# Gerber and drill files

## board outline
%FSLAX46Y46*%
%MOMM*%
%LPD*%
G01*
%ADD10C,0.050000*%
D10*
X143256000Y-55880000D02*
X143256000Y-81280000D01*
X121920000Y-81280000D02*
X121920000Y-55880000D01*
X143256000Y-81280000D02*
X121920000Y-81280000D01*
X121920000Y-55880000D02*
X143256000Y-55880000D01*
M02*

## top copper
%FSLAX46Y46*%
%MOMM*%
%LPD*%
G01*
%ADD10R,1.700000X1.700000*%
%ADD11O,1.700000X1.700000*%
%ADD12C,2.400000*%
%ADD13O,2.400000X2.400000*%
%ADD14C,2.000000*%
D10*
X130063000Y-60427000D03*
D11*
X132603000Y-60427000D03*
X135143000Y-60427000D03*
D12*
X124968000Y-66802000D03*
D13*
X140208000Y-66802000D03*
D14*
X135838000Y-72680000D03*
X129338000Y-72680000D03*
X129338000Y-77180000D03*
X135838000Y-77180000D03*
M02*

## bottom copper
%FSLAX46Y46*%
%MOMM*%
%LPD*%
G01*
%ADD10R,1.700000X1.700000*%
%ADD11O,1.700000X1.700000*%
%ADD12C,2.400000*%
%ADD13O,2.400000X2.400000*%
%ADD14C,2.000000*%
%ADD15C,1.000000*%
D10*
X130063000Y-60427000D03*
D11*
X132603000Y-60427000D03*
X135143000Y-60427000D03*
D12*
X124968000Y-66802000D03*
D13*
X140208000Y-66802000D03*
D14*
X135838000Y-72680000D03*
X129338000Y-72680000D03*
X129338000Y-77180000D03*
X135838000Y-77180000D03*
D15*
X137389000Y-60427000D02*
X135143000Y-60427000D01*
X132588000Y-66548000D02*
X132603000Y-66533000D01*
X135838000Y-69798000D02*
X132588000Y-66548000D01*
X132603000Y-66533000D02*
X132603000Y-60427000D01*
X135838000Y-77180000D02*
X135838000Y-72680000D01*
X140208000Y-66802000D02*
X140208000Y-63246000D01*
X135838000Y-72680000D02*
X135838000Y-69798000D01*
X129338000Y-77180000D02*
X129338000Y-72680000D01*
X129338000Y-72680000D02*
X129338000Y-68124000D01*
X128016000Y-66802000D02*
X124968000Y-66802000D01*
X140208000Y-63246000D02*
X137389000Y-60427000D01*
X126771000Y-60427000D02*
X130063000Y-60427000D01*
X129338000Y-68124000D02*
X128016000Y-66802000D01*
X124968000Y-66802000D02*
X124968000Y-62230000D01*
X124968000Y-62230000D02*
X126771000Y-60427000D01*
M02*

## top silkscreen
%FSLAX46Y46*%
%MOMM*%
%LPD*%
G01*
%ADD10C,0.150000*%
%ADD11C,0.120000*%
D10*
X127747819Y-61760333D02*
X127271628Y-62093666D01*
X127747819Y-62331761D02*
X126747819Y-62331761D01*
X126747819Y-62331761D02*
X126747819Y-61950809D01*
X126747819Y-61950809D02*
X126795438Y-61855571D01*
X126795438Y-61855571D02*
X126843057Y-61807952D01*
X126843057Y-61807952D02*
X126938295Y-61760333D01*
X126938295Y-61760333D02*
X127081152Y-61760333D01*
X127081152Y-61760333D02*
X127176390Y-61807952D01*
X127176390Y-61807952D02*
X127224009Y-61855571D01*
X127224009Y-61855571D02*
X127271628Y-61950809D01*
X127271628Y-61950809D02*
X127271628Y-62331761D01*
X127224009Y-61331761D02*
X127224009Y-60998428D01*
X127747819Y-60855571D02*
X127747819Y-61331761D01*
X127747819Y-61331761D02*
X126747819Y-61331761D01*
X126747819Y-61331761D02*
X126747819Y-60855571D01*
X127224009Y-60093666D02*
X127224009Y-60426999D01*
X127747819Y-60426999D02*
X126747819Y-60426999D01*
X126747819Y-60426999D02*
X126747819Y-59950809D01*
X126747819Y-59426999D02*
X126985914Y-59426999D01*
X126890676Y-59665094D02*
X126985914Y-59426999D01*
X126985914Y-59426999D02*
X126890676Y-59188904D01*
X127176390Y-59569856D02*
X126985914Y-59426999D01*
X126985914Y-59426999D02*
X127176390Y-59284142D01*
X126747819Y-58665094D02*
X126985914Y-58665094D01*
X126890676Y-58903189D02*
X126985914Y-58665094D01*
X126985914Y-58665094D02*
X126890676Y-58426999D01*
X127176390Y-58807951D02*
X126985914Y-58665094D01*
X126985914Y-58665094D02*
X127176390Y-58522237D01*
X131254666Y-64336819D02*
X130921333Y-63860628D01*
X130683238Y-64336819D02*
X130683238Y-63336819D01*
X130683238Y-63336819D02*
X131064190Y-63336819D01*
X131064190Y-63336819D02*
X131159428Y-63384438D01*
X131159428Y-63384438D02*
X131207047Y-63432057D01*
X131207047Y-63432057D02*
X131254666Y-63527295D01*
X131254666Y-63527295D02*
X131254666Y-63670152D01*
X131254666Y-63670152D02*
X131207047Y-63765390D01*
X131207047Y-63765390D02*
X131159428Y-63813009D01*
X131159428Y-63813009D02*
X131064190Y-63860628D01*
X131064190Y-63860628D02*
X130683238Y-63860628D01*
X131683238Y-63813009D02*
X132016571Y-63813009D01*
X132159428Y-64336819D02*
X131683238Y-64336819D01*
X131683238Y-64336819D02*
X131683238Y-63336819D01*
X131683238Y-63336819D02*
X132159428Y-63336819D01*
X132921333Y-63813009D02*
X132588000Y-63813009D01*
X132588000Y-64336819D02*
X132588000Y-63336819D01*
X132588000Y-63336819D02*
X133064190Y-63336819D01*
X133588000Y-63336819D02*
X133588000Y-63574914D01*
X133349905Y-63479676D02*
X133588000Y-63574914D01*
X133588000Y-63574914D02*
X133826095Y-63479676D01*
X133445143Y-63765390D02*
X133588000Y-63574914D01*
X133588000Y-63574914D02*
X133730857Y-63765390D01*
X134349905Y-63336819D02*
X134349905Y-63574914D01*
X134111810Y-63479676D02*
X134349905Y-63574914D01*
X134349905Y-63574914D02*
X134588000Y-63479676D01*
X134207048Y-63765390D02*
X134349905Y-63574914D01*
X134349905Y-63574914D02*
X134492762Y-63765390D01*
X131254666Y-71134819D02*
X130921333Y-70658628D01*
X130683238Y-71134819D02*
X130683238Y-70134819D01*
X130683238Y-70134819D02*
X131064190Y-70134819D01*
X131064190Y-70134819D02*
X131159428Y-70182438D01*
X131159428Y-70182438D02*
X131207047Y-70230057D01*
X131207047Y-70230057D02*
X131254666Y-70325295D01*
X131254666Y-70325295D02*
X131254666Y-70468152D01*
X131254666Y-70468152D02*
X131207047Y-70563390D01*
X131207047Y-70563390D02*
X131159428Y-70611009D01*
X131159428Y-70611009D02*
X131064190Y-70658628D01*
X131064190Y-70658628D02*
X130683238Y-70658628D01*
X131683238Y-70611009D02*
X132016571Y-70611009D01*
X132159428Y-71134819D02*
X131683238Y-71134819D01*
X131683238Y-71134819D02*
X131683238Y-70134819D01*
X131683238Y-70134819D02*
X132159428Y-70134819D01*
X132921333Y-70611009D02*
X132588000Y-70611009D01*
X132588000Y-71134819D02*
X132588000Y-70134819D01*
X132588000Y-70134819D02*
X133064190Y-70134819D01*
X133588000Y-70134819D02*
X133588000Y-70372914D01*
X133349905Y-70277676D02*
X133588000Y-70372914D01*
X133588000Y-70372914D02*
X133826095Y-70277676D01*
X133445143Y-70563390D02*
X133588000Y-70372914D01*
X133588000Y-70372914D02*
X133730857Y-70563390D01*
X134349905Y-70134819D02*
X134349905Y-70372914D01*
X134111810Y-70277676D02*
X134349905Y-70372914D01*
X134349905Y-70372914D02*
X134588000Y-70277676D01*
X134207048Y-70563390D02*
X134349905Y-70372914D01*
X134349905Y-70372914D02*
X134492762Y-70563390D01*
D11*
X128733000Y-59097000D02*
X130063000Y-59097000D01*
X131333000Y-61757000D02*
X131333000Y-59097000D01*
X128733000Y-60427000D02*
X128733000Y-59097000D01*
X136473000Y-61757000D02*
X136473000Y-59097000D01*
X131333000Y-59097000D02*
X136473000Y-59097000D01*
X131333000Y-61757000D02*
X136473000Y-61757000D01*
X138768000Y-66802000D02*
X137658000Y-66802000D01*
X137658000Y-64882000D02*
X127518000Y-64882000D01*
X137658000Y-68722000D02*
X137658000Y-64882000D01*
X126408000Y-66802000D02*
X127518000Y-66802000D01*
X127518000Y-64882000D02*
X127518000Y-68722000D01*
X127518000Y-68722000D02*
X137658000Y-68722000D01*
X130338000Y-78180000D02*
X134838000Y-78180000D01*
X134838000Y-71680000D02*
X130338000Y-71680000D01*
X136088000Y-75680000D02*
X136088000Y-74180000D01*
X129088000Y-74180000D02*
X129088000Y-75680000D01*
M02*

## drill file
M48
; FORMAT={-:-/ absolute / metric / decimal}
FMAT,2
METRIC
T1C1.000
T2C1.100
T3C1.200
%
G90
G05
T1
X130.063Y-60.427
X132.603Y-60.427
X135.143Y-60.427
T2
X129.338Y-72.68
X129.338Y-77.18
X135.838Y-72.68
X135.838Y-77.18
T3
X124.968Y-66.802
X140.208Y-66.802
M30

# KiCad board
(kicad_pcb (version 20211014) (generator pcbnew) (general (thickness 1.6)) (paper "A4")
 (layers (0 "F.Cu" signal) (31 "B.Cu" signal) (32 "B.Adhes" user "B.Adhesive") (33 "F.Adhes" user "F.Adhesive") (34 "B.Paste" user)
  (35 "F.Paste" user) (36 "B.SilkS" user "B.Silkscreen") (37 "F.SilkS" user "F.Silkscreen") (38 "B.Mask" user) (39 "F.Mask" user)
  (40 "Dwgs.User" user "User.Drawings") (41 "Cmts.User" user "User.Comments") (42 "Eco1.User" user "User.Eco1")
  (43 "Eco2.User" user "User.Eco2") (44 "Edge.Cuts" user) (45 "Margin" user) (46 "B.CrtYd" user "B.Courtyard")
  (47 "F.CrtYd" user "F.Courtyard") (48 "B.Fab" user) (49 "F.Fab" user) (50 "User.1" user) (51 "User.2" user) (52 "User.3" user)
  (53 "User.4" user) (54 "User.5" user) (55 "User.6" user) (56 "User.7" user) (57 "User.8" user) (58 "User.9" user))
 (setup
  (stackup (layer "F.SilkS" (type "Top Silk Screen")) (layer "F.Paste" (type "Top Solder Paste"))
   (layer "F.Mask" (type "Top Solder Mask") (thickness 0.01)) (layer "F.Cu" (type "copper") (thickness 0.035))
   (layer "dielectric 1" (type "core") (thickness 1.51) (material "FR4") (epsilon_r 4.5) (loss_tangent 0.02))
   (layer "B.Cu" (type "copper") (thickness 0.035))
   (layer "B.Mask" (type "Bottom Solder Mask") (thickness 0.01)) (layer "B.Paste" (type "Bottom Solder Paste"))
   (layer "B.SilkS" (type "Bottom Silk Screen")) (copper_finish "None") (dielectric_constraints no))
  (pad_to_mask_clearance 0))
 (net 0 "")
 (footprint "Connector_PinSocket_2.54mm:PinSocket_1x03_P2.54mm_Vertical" (layer "F.Cu") (at 130.063 60.427 90)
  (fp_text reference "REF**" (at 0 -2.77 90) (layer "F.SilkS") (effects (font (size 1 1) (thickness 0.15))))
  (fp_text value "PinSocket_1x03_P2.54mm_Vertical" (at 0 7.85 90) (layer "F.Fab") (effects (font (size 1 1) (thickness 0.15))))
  (fp_line (start 1.33 -1.33) (end 1.33 0) (layer "F.SilkS") (width 0.12))
  (fp_line (start -1.33 1.27) (end 1.33 1.27) (layer "F.SilkS") (width 0.12))
  (fp_line (start 0 -1.33) (end 1.33 -1.33) (layer "F.SilkS") (width 0.12))
  (fp_line (start -1.33 6.41) (end 1.33 6.41) (layer "F.SilkS") (width 0.12))
  (fp_line (start 1.33 1.27) (end 1.33 6.41) (layer "F.SilkS") (width 0.12))
  (fp_line (start -1.33 1.27) (end -1.33 6.41) (layer "F.SilkS") (width 0.12))
  (pad "1" thru_hole rect (at 0 0 90) (size 1.7 1.7) (drill 1) (layers *.Cu *.Mask))
  (pad "2" thru_hole oval (at 0 2.54 90) (size 1.7 1.7) (drill 1) (layers *.Cu *.Mask))
  (pad "3" thru_hole oval (at 0 5.08 90) (size 1.7 1.7) (drill 1) (layers *.Cu *.Mask)))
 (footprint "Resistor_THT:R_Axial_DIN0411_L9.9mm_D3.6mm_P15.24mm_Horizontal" (layer "F.Cu") (at 124.968 66.802)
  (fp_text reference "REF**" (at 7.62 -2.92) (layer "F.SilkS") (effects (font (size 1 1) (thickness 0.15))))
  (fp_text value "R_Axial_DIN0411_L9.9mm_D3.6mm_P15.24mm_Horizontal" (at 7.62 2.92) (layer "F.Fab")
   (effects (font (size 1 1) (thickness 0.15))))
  (fp_line (start 13.8 0) (end 12.69 0) (layer "F.SilkS") (width 0.12))
  (fp_line (start 12.69 -1.92) (end 2.55 -1.92) (layer "F.SilkS") (width 0.12))
  (fp_line (start 12.69 1.92) (end 12.69 -1.92) (layer "F.SilkS") (width 0.12))
  (fp_line (start 1.44 0) (end 2.55 0) (layer "F.SilkS") (width 0.12))
  (fp_line (start 2.55 -1.92) (end 2.55 1.92) (layer "F.SilkS") (width 0.12))
  (fp_line (start 2.55 1.92) (end 12.69 1.92) (layer "F.SilkS") (width 0.12))
  (pad "1" thru_hole circle (at 0 0) (size 2.4 2.4) (drill 1.2) (layers *.Cu *.Mask))
  (pad "2" thru_hole oval (at 15.24 0) (size 2.4 2.4) (drill 1.2) (layers *.Cu *.Mask)))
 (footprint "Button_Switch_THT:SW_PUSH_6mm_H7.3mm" (layer "F.Cu") (at 129.338 72.68)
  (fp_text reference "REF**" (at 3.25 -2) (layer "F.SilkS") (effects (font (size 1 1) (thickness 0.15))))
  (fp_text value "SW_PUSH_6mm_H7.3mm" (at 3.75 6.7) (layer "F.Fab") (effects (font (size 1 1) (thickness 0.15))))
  (fp_line (start 1 5.5) (end 5.5 5.5) (layer "F.SilkS") (width 0.12))
  (fp_line (start 5.5 -1) (end 1 -1) (layer "F.SilkS") (width 0.12))
  (fp_line (start 6.75 3) (end 6.75 1.5) (layer "F.SilkS") (width 0.12))
  (fp_line (start -0.25 1.5) (end -0.25 3) (layer "F.SilkS") (width 0.12))
  (pad "1" thru_hole circle (at 6.5 0 90) (size 2 2) (drill 1.1) (layers *.Cu *.Mask))
  (pad "1" thru_hole circle (at 0 0 90) (size 2 2) (drill 1.1) (layers *.Cu *.Mask))
  (pad "2" thru_hole circle (at 0 4.5 90) (size 2 2) (drill 1.1) (layers *.Cu *.Mask))
  (pad "2" thru_hole circle (at 6.5 4.5 90) (size 2 2) (drill 1.1) (layers *.Cu *.Mask)))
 (gr_line (start 143.256 55.88) (end 143.256 81.28) (layer "Edge.Cuts") (width 0.05))
 (gr_line (start 121.92 81.28) (end 121.92 55.88) (layer "Edge.Cuts") (width 0.05))
 (gr_line (start 143.256 81.28) (end 121.92 81.28) (layer "Edge.Cuts") (width 0.05))
 (gr_line (start 121.92 55.88) (end 143.256 55.88) (layer "Edge.Cuts") (width 0.05))
 (segment (start 137.389 60.427) (end 135.143 60.427) (width 1) (layer "B.Cu") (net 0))
 (segment (start 132.588 66.548) (end 132.603 66.533) (width 1) (layer "B.Cu") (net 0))
 (segment (start 135.838 69.798) (end 132.588 66.548) (width 1) (layer "B.Cu") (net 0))
 (segment (start 132.603 66.533) (end 132.603 60.427) (width 1) (layer "B.Cu") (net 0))
 (segment (start 135.838 77.18) (end 135.838 72.68) (width 1) (layer "B.Cu") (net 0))
 (segment (start 140.208 66.802) (end 140.208 63.246) (width 1) (layer "B.Cu") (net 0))
 (segment (start 135.838 72.68) (end 135.838 69.798) (width 1) (layer "B.Cu") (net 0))
 (segment (start 129.338 77.18) (end 129.338 72.68) (width 1) (layer "B.Cu") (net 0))
 (segment (start 129.338 72.68) (end 129.338 68.124) (width 1) (layer "B.Cu") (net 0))
 (segment (start 128.016 66.802) (end 124.968 66.802) (width 1) (layer "B.Cu") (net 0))
 (segment (start 140.208 63.246) (end 137.389 60.427) (width 1) (layer "B.Cu") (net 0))
 (segment (start 126.771 60.427) (end 130.063 60.427) (width 1) (layer "B.Cu") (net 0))
 (segment (start 129.338 68.124) (end 128.016 66.802) (width 1) (layer "B.Cu") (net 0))
 (segment (start 124.968 66.802) (end 124.968 62.23) (width 1) (layer "B.Cu") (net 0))
 (segment (start 124.968 62.23) (end 126.771 60.427) (width 1) (layer "B.Cu") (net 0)))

